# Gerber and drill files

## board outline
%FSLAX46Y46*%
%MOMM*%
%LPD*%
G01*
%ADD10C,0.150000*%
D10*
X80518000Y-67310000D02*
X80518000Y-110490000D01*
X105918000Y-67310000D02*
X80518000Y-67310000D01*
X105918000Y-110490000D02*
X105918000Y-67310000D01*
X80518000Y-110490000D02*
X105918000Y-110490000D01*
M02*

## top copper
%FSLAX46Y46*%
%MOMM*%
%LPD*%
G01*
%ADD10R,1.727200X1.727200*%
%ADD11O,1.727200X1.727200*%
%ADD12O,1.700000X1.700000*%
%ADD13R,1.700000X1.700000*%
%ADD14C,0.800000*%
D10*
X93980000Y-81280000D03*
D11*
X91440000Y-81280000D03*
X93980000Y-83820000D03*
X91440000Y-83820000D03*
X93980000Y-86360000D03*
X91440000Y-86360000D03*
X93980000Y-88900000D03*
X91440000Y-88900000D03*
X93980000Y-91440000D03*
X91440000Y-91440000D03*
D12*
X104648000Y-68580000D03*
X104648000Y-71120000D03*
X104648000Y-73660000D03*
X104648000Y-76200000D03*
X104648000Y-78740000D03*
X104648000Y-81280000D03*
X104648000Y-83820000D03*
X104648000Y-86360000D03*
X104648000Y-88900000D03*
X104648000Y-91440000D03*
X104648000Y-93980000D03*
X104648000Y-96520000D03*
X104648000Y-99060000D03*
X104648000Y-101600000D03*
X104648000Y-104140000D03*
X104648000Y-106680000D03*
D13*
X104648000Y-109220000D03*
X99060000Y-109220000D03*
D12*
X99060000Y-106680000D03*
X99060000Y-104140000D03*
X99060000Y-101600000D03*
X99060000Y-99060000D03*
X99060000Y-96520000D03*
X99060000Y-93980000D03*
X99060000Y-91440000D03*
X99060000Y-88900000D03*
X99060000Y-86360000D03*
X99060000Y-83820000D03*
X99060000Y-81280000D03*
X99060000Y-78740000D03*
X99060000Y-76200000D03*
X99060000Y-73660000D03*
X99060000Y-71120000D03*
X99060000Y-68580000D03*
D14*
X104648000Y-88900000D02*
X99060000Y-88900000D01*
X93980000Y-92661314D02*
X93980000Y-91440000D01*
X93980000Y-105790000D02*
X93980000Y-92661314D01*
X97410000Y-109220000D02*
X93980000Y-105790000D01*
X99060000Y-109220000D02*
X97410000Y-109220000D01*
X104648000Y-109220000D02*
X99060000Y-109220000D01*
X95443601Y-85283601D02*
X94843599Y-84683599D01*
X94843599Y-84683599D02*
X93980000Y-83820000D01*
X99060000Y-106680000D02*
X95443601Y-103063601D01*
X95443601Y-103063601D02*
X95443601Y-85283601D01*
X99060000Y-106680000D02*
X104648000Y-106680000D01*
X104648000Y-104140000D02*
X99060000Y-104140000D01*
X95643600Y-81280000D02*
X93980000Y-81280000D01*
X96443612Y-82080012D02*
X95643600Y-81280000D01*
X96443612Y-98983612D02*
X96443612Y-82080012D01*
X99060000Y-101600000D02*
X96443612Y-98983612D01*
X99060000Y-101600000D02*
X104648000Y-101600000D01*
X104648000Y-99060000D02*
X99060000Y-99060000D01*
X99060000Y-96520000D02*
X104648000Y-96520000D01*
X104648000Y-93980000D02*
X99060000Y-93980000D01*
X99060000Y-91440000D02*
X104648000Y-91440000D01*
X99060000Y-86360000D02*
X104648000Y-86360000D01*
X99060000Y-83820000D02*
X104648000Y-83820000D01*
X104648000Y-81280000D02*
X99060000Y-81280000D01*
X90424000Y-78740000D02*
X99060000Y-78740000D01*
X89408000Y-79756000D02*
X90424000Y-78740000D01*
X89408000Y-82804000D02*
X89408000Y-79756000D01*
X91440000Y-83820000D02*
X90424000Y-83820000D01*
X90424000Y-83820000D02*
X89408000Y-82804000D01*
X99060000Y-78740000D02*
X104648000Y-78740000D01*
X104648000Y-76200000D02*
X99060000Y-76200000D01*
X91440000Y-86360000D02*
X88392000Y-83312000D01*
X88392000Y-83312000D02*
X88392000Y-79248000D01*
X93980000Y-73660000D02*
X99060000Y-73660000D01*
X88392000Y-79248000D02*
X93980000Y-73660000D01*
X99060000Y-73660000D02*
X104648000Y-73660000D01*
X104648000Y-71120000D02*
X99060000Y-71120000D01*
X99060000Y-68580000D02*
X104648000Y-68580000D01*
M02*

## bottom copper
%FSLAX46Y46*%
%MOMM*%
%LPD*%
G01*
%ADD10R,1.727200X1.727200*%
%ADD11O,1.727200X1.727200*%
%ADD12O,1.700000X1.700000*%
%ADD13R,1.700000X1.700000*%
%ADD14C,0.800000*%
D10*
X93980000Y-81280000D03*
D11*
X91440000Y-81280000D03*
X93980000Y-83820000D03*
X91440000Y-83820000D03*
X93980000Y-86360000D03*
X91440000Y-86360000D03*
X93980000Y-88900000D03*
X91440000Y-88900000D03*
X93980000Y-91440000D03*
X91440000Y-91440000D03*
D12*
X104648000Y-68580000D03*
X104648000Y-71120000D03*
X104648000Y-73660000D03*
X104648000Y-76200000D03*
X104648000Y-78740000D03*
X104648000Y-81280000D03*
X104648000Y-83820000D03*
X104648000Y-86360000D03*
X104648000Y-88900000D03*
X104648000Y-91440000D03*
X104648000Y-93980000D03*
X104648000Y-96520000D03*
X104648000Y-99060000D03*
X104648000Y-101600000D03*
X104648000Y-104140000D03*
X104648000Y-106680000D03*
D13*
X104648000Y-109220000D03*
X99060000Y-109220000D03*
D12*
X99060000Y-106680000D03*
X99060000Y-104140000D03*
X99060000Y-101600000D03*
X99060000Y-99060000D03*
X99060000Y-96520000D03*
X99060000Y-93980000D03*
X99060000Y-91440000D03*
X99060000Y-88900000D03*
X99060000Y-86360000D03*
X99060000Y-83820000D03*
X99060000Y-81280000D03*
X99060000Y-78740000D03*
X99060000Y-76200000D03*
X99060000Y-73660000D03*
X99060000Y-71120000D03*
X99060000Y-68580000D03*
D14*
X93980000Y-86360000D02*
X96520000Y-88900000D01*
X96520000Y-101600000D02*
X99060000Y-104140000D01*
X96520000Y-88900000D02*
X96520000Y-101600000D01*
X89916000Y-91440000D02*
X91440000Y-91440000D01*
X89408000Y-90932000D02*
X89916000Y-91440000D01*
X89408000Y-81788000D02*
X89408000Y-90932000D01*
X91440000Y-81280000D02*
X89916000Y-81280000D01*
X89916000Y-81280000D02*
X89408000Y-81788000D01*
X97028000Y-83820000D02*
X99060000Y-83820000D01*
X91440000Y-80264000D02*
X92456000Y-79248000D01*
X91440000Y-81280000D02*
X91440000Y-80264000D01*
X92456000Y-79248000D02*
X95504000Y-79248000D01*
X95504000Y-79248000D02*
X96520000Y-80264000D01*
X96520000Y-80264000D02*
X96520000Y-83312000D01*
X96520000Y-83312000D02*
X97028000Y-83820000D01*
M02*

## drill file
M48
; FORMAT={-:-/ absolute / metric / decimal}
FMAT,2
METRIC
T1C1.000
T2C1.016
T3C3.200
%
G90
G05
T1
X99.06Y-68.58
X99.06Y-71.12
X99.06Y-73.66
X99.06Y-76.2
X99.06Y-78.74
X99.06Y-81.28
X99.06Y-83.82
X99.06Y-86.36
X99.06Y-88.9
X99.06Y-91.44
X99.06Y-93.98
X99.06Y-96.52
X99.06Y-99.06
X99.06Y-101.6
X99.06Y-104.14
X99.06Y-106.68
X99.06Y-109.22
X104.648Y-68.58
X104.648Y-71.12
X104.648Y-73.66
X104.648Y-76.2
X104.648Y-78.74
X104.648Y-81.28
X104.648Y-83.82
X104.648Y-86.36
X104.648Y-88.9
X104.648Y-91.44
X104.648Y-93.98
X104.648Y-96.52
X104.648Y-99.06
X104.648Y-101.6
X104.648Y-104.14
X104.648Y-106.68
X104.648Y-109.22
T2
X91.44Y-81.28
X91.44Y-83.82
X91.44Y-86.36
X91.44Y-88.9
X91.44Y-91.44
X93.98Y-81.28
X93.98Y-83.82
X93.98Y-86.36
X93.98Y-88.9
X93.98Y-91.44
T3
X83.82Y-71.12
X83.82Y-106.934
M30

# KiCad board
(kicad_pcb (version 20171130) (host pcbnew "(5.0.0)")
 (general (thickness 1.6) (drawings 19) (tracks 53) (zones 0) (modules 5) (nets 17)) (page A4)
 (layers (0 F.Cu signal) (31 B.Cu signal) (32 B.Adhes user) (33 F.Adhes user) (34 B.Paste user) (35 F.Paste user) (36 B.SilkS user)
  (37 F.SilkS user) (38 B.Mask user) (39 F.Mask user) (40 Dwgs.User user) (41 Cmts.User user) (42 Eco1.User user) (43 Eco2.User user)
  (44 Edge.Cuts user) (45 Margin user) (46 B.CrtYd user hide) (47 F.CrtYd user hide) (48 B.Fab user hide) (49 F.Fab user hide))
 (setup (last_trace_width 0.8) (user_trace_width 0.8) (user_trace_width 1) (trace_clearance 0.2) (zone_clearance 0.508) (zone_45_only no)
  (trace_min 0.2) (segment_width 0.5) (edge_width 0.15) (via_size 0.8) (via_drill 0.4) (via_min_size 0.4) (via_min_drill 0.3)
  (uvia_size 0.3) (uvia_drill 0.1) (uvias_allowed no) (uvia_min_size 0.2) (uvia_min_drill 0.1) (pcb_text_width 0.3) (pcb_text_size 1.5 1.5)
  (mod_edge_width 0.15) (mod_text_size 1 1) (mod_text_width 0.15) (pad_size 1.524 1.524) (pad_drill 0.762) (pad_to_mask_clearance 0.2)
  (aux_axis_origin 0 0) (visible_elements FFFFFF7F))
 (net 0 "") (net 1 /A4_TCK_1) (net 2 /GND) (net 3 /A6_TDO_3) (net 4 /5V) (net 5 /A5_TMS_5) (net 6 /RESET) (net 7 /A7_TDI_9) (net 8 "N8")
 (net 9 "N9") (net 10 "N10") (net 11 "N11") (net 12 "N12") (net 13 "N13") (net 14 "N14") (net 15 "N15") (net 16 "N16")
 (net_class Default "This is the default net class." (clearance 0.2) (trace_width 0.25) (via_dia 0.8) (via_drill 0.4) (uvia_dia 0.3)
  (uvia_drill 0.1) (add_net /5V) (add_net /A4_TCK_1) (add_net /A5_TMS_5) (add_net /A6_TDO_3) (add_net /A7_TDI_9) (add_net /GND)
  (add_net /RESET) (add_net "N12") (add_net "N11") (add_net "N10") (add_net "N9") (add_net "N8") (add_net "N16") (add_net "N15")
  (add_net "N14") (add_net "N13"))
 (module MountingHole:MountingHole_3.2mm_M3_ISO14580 (layer F.Cu) (at 83.82 71.12)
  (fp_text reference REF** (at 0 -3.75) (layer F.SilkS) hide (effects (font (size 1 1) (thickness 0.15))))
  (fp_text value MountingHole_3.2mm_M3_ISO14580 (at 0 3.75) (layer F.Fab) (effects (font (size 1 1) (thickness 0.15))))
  (pad 1 np_thru_hole circle (at 0 0) (size 3.2 3.2) (drill 3.2) (layers *.Cu *.Mask)))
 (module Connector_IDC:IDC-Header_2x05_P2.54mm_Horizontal (layer B.Cu) (at 93.98 81.28 180)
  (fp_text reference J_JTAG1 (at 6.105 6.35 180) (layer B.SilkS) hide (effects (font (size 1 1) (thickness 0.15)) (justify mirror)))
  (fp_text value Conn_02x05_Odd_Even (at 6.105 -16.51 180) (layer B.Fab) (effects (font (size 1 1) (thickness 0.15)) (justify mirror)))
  (pad 1 thru_hole rect (at 0 0 180) (size 1.7272 1.7272) (drill 1.016) (layers *.Cu *.Mask) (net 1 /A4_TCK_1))
  (pad 2 thru_hole oval (at 2.54 0 180) (size 1.7272 1.7272) (drill 1.016) (layers *.Cu *.Mask) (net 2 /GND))
  (pad 3 thru_hole oval (at 0 -2.54 180) (size 1.7272 1.7272) (drill 1.016) (layers *.Cu *.Mask) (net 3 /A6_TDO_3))
  (pad 4 thru_hole oval (at 2.54 -2.54 180) (size 1.7272 1.7272) (drill 1.016) (layers *.Cu *.Mask) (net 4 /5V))
  (pad 5 thru_hole oval (at 0 -5.08 180) (size 1.7272 1.7272) (drill 1.016) (layers *.Cu *.Mask) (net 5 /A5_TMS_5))
  (pad 6 thru_hole oval (at 2.54 -5.08 180) (size 1.7272 1.7272) (drill 1.016) (layers *.Cu *.Mask) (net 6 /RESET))
  (pad 7 thru_hole oval (at 0 -7.62 180) (size 1.7272 1.7272) (drill 1.016) (layers *.Cu *.Mask))
  (pad 8 thru_hole oval (at 2.54 -7.62 180) (size 1.7272 1.7272) (drill 1.016) (layers *.Cu *.Mask))
  (pad 9 thru_hole oval (at 0 -10.16 180) (size 1.7272 1.7272) (drill 1.016) (layers *.Cu *.Mask) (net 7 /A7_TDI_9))
  (pad 10 thru_hole oval (at 2.54 -10.16 180) (size 1.7272 1.7272) (drill 1.016) (layers *.Cu *.Mask) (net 2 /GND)))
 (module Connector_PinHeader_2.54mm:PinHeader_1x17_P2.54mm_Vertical (layer B.Cu) (at 104.648 109.22)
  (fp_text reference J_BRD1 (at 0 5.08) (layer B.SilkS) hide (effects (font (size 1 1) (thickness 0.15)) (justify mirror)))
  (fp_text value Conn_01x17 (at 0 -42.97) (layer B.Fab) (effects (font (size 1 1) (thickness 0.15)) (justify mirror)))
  (pad 17 thru_hole oval (at 0 -40.64) (size 1.7 1.7) (drill 1) (layers *.Cu *.Mask) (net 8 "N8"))
  (pad 16 thru_hole oval (at 0 -38.1) (size 1.7 1.7) (drill 1) (layers *.Cu *.Mask) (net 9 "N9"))
  (pad 15 thru_hole oval (at 0 -35.56) (size 1.7 1.7) (drill 1) (layers *.Cu *.Mask) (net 6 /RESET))
  (pad 14 thru_hole oval (at 0 -33.02) (size 1.7 1.7) (drill 1) (layers *.Cu *.Mask) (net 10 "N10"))
  (pad 13 thru_hole oval (at 0 -30.48) (size 1.7 1.7) (drill 1) (layers *.Cu *.Mask) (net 4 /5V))
  (pad 12 thru_hole oval (at 0 -27.94) (size 1.7 1.7) (drill 1) (layers *.Cu *.Mask) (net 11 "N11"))
  (pad 11 thru_hole oval (at 0 -25.4) (size 1.7 1.7) (drill 1) (layers *.Cu *.Mask) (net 2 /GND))
  (pad 10 thru_hole oval (at 0 -22.86) (size 1.7 1.7) (drill 1) (layers *.Cu *.Mask) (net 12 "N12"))
  (pad 9 thru_hole oval (at 0 -20.32) (size 1.7 1.7) (drill 1) (layers *.Cu *.Mask))
  (pad 8 thru_hole oval (at 0 -17.78) (size 1.7 1.7) (drill 1) (layers *.Cu *.Mask) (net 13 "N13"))
  (pad 7 thru_hole oval (at 0 -15.24) (size 1.7 1.7) (drill 1) (layers *.Cu *.Mask) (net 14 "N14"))
  (pad 6 thru_hole oval (at 0 -12.7) (size 1.7 1.7) (drill 1) (layers *.Cu *.Mask) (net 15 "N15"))
  (pad 5 thru_hole oval (at 0 -10.16) (size 1.7 1.7) (drill 1) (layers *.Cu *.Mask) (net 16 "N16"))
  (pad 4 thru_hole oval (at 0 -7.62) (size 1.7 1.7) (drill 1) (layers *.Cu *.Mask) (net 1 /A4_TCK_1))
  (pad 3 thru_hole oval (at 0 -5.08) (size 1.7 1.7) (drill 1) (layers *.Cu *.Mask) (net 5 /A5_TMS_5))
  (pad 2 thru_hole oval (at 0 -2.54) (size 1.7 1.7) (drill 1) (layers *.Cu *.Mask) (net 3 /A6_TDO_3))
  (pad 1 thru_hole rect (at 0 0) (size 1.7 1.7) (drill 1) (layers *.Cu *.Mask) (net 7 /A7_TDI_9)))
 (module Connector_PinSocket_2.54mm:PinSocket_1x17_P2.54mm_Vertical (layer F.Cu) (at 99.06 109.22 180)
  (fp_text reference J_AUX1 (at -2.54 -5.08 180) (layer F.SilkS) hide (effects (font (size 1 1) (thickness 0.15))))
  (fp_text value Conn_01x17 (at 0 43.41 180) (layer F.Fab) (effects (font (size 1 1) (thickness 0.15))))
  (pad 1 thru_hole rect (at 0 0 180) (size 1.7 1.7) (drill 1) (layers *.Cu *.Mask) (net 7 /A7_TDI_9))
  (pad 2 thru_hole oval (at 0 2.54 180) (size 1.7 1.7) (drill 1) (layers *.Cu *.Mask) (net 3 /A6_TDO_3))
  (pad 3 thru_hole oval (at 0 5.08 180) (size 1.7 1.7) (drill 1) (layers *.Cu *.Mask) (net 5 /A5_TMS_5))
  (pad 4 thru_hole oval (at 0 7.62 180) (size 1.7 1.7) (drill 1) (layers *.Cu *.Mask) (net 1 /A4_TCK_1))
  (pad 5 thru_hole oval (at 0 10.16 180) (size 1.7 1.7) (drill 1) (layers *.Cu *.Mask) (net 16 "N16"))
  (pad 6 thru_hole oval (at 0 12.7 180) (size 1.7 1.7) (drill 1) (layers *.Cu *.Mask) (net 15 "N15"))
  (pad 7 thru_hole oval (at 0 15.24 180) (size 1.7 1.7) (drill 1) (layers *.Cu *.Mask) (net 14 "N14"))
  (pad 8 thru_hole oval (at 0 17.78 180) (size 1.7 1.7) (drill 1) (layers *.Cu *.Mask) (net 13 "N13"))
  (pad 9 thru_hole oval (at 0 20.32 180) (size 1.7 1.7) (drill 1) (layers *.Cu *.Mask))
  (pad 10 thru_hole oval (at 0 22.86 180) (size 1.7 1.7) (drill 1) (layers *.Cu *.Mask) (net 12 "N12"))
  (pad 11 thru_hole oval (at 0 25.4 180) (size 1.7 1.7) (drill 1) (layers *.Cu *.Mask) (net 2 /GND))
  (pad 12 thru_hole oval (at 0 27.94 180) (size 1.7 1.7) (drill 1) (layers *.Cu *.Mask) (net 11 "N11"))
  (pad 13 thru_hole oval (at 0 30.48 180) (size 1.7 1.7) (drill 1) (layers *.Cu *.Mask) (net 4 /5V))
  (pad 14 thru_hole oval (at 0 33.02 180) (size 1.7 1.7) (drill 1) (layers *.Cu *.Mask) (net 10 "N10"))
  (pad 15 thru_hole oval (at 0 35.56 180) (size 1.7 1.7) (drill 1) (layers *.Cu *.Mask) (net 6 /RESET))
  (pad 16 thru_hole oval (at 0 38.1 180) (size 1.7 1.7) (drill 1) (layers *.Cu *.Mask) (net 9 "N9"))
  (pad 17 thru_hole oval (at 0 40.64 180) (size 1.7 1.7) (drill 1) (layers *.Cu *.Mask) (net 8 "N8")))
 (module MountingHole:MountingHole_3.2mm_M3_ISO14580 (layer F.Cu) (at 83.82 106.934)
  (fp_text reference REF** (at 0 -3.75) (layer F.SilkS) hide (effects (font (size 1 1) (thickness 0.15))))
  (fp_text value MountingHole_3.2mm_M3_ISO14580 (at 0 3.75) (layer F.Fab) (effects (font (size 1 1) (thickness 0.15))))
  (pad 1 np_thru_hole circle (at 0 0) (size 3.2 3.2) (drill 3.2) (layers *.Cu *.Mask)))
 (gr_line (start 80.518 67.31) (end 80.518 110.49) (layer Edge.Cuts) (width 0.15))
 (gr_line (start 105.918 67.31) (end 80.518 67.31) (layer Edge.Cuts) (width 0.15))
 (gr_line (start 105.918 110.49) (end 105.918 67.31) (layer Edge.Cuts) (width 0.15))
 (gr_line (start 80.518 110.49) (end 105.918 110.49) (layer Edge.Cuts) (width 0.15))
 (segment (start 104.648 88.9) (end 99.06 88.9) (width 0.8) (layer F.Cu) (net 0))
 (segment (start 93.98 92.661314) (end 93.98 91.44) (width 0.8) (layer F.Cu) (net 7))
 (segment (start 93.98 105.79) (end 93.98 92.661314) (width 0.8) (layer F.Cu) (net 7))
 (segment (start 97.41 109.22) (end 93.98 105.79) (width 0.8) (layer F.Cu) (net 7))
 (segment (start 99.06 109.22) (end 97.41 109.22) (width 0.8) (layer F.Cu) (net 7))
 (segment (start 104.648 109.22) (end 99.06 109.22) (width 0.8) (layer F.Cu) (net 7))
 (segment (start 95.443601 85.283601) (end 94.843599 84.683599) (width 0.8) (layer F.Cu) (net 3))
 (segment (start 94.843599 84.683599) (end 93.98 83.82) (width 0.8) (layer F.Cu) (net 3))
 (segment (start 99.06 106.68) (end 95.443601 103.063601) (width 0.8) (layer F.Cu) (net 3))
 (segment (start 95.443601 103.063601) (end 95.443601 85.283601) (width 0.8) (layer F.Cu) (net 3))
 (segment (start 99.06 106.68) (end 104.648 106.68) (width 0.8) (layer F.Cu) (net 3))
 (segment (start 93.98 86.36) (end 96.52 88.9) (width 0.8) (layer B.Cu) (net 5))
 (segment (start 96.52 101.6) (end 99.06 104.14) (width 0.8) (layer B.Cu) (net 5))
 (segment (start 96.52 88.9) (end 96.52 101.6) (width 0.8) (layer B.Cu) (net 5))
 (segment (start 104.648 104.14) (end 99.06 104.14) (width 0.8) (layer F.Cu) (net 5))
 (segment (start 95.6436 81.28) (end 93.98 81.28) (width 0.8) (layer F.Cu) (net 1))
 (segment (start 96.443612 82.080012) (end 95.6436 81.28) (width 0.8) (layer F.Cu) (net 1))
 (segment (start 96.443612 98.983612) (end 96.443612 82.080012) (width 0.8) (layer F.Cu) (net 1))
 (segment (start 99.06 101.6) (end 96.443612 98.983612) (width 0.8) (layer F.Cu) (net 1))
 (segment (start 99.06 101.6) (end 104.648 101.6) (width 0.8) (layer F.Cu) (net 1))
 (segment (start 104.648 99.06) (end 99.06 99.06) (width 0.8) (layer F.Cu) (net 16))
 (segment (start 99.06 96.52) (end 104.648 96.52) (width 0.8) (layer F.Cu) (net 15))
 (segment (start 104.648 93.98) (end 99.06 93.98) (width 0.8) (layer F.Cu) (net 14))
 (segment (start 99.06 91.44) (end 104.648 91.44) (width 0.8) (layer F.Cu) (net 13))
 (segment (start 99.06 86.36) (end 104.648 86.36) (width 0.8) (layer F.Cu) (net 12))
 (segment (start 89.916 91.44) (end 91.44 91.44) (width 0.8) (layer B.Cu) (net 2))
 (segment (start 89.408 90.932) (end 89.916 91.44) (width 0.8) (layer B.Cu) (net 2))
 (segment (start 89.408 81.788) (end 89.408 90.932) (width 0.8) (layer B.Cu) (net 2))
 (segment (start 91.44 81.28) (end 89.916 81.28) (width 0.8) (layer B.Cu) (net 2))
 (segment (start 89.916 81.28) (end 89.408 81.788) (width 0.8) (layer B.Cu) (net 2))
 (segment (start 97.028 83.82) (end 99.06 83.82) (width 0.8) (layer B.Cu) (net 2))
 (segment (start 91.44 80.264) (end 92.456 79.248) (width 0.8) (layer B.Cu) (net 2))
 (segment (start 91.44 81.28) (end 91.44 80.264) (width 0.8) (layer B.Cu) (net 2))
 (segment (start 92.456 79.248) (end 95.504 79.248) (width 0.8) (layer B.Cu) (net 2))
 (segment (start 95.504 79.248) (end 96.52 80.264) (width 0.8) (layer B.Cu) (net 2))
 (segment (start 96.52 80.264) (end 96.52 83.312) (width 0.8) (layer B.Cu) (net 2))
 (segment (start 96.52 83.312) (end 97.028 83.82) (width 0.8) (layer B.Cu) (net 2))
 (segment (start 99.06 83.82) (end 104.648 83.82) (width 0.8) (layer F.Cu) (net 2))
 (segment (start 104.648 81.28) (end 99.06 81.28) (width 0.8) (layer F.Cu) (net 11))
 (segment (start 90.424 78.74) (end 99.06 78.74) (width 0.8) (layer F.Cu) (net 4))
 (segment (start 89.408 79.756) (end 90.424 78.74) (width 0.8) (layer F.Cu) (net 4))
 (segment (start 89.408 82.804) (end 89.408 79.756) (width 0.8) (layer F.Cu) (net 4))
 (segment (start 91.44 83.82) (end 90.424 83.82) (width 0.8) (layer F.Cu) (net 4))
 (segment (start 90.424 83.82) (end 89.408 82.804) (width 0.8) (layer F.Cu) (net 4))
 (segment (start 99.06 78.74) (end 104.648 78.74) (width 0.8) (layer F.Cu) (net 4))
 (segment (start 104.648 76.2) (end 99.06 76.2) (width 0.8) (layer F.Cu) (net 10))
 (segment (start 91.44 86.36) (end 88.392 83.312) (width 0.8) (layer F.Cu) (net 6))
 (segment (start 88.392 83.312) (end 88.392 79.248) (width 0.8) (layer F.Cu) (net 6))
 (segment (start 93.98 73.66) (end 99.06 73.66) (width 0.8) (layer F.Cu) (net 6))
 (segment (start 88.392 79.248) (end 93.98 73.66) (width 0.8) (layer F.Cu) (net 6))
 (segment (start 99.06 73.66) (end 104.648 73.66) (width 0.8) (layer F.Cu) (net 6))
 (segment (start 104.648 71.12) (end 99.06 71.12) (width 0.8) (layer F.Cu) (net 9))
 (segment (start 99.06 68.58) (end 104.648 68.58) (width 0.8) (layer F.Cu) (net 8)))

